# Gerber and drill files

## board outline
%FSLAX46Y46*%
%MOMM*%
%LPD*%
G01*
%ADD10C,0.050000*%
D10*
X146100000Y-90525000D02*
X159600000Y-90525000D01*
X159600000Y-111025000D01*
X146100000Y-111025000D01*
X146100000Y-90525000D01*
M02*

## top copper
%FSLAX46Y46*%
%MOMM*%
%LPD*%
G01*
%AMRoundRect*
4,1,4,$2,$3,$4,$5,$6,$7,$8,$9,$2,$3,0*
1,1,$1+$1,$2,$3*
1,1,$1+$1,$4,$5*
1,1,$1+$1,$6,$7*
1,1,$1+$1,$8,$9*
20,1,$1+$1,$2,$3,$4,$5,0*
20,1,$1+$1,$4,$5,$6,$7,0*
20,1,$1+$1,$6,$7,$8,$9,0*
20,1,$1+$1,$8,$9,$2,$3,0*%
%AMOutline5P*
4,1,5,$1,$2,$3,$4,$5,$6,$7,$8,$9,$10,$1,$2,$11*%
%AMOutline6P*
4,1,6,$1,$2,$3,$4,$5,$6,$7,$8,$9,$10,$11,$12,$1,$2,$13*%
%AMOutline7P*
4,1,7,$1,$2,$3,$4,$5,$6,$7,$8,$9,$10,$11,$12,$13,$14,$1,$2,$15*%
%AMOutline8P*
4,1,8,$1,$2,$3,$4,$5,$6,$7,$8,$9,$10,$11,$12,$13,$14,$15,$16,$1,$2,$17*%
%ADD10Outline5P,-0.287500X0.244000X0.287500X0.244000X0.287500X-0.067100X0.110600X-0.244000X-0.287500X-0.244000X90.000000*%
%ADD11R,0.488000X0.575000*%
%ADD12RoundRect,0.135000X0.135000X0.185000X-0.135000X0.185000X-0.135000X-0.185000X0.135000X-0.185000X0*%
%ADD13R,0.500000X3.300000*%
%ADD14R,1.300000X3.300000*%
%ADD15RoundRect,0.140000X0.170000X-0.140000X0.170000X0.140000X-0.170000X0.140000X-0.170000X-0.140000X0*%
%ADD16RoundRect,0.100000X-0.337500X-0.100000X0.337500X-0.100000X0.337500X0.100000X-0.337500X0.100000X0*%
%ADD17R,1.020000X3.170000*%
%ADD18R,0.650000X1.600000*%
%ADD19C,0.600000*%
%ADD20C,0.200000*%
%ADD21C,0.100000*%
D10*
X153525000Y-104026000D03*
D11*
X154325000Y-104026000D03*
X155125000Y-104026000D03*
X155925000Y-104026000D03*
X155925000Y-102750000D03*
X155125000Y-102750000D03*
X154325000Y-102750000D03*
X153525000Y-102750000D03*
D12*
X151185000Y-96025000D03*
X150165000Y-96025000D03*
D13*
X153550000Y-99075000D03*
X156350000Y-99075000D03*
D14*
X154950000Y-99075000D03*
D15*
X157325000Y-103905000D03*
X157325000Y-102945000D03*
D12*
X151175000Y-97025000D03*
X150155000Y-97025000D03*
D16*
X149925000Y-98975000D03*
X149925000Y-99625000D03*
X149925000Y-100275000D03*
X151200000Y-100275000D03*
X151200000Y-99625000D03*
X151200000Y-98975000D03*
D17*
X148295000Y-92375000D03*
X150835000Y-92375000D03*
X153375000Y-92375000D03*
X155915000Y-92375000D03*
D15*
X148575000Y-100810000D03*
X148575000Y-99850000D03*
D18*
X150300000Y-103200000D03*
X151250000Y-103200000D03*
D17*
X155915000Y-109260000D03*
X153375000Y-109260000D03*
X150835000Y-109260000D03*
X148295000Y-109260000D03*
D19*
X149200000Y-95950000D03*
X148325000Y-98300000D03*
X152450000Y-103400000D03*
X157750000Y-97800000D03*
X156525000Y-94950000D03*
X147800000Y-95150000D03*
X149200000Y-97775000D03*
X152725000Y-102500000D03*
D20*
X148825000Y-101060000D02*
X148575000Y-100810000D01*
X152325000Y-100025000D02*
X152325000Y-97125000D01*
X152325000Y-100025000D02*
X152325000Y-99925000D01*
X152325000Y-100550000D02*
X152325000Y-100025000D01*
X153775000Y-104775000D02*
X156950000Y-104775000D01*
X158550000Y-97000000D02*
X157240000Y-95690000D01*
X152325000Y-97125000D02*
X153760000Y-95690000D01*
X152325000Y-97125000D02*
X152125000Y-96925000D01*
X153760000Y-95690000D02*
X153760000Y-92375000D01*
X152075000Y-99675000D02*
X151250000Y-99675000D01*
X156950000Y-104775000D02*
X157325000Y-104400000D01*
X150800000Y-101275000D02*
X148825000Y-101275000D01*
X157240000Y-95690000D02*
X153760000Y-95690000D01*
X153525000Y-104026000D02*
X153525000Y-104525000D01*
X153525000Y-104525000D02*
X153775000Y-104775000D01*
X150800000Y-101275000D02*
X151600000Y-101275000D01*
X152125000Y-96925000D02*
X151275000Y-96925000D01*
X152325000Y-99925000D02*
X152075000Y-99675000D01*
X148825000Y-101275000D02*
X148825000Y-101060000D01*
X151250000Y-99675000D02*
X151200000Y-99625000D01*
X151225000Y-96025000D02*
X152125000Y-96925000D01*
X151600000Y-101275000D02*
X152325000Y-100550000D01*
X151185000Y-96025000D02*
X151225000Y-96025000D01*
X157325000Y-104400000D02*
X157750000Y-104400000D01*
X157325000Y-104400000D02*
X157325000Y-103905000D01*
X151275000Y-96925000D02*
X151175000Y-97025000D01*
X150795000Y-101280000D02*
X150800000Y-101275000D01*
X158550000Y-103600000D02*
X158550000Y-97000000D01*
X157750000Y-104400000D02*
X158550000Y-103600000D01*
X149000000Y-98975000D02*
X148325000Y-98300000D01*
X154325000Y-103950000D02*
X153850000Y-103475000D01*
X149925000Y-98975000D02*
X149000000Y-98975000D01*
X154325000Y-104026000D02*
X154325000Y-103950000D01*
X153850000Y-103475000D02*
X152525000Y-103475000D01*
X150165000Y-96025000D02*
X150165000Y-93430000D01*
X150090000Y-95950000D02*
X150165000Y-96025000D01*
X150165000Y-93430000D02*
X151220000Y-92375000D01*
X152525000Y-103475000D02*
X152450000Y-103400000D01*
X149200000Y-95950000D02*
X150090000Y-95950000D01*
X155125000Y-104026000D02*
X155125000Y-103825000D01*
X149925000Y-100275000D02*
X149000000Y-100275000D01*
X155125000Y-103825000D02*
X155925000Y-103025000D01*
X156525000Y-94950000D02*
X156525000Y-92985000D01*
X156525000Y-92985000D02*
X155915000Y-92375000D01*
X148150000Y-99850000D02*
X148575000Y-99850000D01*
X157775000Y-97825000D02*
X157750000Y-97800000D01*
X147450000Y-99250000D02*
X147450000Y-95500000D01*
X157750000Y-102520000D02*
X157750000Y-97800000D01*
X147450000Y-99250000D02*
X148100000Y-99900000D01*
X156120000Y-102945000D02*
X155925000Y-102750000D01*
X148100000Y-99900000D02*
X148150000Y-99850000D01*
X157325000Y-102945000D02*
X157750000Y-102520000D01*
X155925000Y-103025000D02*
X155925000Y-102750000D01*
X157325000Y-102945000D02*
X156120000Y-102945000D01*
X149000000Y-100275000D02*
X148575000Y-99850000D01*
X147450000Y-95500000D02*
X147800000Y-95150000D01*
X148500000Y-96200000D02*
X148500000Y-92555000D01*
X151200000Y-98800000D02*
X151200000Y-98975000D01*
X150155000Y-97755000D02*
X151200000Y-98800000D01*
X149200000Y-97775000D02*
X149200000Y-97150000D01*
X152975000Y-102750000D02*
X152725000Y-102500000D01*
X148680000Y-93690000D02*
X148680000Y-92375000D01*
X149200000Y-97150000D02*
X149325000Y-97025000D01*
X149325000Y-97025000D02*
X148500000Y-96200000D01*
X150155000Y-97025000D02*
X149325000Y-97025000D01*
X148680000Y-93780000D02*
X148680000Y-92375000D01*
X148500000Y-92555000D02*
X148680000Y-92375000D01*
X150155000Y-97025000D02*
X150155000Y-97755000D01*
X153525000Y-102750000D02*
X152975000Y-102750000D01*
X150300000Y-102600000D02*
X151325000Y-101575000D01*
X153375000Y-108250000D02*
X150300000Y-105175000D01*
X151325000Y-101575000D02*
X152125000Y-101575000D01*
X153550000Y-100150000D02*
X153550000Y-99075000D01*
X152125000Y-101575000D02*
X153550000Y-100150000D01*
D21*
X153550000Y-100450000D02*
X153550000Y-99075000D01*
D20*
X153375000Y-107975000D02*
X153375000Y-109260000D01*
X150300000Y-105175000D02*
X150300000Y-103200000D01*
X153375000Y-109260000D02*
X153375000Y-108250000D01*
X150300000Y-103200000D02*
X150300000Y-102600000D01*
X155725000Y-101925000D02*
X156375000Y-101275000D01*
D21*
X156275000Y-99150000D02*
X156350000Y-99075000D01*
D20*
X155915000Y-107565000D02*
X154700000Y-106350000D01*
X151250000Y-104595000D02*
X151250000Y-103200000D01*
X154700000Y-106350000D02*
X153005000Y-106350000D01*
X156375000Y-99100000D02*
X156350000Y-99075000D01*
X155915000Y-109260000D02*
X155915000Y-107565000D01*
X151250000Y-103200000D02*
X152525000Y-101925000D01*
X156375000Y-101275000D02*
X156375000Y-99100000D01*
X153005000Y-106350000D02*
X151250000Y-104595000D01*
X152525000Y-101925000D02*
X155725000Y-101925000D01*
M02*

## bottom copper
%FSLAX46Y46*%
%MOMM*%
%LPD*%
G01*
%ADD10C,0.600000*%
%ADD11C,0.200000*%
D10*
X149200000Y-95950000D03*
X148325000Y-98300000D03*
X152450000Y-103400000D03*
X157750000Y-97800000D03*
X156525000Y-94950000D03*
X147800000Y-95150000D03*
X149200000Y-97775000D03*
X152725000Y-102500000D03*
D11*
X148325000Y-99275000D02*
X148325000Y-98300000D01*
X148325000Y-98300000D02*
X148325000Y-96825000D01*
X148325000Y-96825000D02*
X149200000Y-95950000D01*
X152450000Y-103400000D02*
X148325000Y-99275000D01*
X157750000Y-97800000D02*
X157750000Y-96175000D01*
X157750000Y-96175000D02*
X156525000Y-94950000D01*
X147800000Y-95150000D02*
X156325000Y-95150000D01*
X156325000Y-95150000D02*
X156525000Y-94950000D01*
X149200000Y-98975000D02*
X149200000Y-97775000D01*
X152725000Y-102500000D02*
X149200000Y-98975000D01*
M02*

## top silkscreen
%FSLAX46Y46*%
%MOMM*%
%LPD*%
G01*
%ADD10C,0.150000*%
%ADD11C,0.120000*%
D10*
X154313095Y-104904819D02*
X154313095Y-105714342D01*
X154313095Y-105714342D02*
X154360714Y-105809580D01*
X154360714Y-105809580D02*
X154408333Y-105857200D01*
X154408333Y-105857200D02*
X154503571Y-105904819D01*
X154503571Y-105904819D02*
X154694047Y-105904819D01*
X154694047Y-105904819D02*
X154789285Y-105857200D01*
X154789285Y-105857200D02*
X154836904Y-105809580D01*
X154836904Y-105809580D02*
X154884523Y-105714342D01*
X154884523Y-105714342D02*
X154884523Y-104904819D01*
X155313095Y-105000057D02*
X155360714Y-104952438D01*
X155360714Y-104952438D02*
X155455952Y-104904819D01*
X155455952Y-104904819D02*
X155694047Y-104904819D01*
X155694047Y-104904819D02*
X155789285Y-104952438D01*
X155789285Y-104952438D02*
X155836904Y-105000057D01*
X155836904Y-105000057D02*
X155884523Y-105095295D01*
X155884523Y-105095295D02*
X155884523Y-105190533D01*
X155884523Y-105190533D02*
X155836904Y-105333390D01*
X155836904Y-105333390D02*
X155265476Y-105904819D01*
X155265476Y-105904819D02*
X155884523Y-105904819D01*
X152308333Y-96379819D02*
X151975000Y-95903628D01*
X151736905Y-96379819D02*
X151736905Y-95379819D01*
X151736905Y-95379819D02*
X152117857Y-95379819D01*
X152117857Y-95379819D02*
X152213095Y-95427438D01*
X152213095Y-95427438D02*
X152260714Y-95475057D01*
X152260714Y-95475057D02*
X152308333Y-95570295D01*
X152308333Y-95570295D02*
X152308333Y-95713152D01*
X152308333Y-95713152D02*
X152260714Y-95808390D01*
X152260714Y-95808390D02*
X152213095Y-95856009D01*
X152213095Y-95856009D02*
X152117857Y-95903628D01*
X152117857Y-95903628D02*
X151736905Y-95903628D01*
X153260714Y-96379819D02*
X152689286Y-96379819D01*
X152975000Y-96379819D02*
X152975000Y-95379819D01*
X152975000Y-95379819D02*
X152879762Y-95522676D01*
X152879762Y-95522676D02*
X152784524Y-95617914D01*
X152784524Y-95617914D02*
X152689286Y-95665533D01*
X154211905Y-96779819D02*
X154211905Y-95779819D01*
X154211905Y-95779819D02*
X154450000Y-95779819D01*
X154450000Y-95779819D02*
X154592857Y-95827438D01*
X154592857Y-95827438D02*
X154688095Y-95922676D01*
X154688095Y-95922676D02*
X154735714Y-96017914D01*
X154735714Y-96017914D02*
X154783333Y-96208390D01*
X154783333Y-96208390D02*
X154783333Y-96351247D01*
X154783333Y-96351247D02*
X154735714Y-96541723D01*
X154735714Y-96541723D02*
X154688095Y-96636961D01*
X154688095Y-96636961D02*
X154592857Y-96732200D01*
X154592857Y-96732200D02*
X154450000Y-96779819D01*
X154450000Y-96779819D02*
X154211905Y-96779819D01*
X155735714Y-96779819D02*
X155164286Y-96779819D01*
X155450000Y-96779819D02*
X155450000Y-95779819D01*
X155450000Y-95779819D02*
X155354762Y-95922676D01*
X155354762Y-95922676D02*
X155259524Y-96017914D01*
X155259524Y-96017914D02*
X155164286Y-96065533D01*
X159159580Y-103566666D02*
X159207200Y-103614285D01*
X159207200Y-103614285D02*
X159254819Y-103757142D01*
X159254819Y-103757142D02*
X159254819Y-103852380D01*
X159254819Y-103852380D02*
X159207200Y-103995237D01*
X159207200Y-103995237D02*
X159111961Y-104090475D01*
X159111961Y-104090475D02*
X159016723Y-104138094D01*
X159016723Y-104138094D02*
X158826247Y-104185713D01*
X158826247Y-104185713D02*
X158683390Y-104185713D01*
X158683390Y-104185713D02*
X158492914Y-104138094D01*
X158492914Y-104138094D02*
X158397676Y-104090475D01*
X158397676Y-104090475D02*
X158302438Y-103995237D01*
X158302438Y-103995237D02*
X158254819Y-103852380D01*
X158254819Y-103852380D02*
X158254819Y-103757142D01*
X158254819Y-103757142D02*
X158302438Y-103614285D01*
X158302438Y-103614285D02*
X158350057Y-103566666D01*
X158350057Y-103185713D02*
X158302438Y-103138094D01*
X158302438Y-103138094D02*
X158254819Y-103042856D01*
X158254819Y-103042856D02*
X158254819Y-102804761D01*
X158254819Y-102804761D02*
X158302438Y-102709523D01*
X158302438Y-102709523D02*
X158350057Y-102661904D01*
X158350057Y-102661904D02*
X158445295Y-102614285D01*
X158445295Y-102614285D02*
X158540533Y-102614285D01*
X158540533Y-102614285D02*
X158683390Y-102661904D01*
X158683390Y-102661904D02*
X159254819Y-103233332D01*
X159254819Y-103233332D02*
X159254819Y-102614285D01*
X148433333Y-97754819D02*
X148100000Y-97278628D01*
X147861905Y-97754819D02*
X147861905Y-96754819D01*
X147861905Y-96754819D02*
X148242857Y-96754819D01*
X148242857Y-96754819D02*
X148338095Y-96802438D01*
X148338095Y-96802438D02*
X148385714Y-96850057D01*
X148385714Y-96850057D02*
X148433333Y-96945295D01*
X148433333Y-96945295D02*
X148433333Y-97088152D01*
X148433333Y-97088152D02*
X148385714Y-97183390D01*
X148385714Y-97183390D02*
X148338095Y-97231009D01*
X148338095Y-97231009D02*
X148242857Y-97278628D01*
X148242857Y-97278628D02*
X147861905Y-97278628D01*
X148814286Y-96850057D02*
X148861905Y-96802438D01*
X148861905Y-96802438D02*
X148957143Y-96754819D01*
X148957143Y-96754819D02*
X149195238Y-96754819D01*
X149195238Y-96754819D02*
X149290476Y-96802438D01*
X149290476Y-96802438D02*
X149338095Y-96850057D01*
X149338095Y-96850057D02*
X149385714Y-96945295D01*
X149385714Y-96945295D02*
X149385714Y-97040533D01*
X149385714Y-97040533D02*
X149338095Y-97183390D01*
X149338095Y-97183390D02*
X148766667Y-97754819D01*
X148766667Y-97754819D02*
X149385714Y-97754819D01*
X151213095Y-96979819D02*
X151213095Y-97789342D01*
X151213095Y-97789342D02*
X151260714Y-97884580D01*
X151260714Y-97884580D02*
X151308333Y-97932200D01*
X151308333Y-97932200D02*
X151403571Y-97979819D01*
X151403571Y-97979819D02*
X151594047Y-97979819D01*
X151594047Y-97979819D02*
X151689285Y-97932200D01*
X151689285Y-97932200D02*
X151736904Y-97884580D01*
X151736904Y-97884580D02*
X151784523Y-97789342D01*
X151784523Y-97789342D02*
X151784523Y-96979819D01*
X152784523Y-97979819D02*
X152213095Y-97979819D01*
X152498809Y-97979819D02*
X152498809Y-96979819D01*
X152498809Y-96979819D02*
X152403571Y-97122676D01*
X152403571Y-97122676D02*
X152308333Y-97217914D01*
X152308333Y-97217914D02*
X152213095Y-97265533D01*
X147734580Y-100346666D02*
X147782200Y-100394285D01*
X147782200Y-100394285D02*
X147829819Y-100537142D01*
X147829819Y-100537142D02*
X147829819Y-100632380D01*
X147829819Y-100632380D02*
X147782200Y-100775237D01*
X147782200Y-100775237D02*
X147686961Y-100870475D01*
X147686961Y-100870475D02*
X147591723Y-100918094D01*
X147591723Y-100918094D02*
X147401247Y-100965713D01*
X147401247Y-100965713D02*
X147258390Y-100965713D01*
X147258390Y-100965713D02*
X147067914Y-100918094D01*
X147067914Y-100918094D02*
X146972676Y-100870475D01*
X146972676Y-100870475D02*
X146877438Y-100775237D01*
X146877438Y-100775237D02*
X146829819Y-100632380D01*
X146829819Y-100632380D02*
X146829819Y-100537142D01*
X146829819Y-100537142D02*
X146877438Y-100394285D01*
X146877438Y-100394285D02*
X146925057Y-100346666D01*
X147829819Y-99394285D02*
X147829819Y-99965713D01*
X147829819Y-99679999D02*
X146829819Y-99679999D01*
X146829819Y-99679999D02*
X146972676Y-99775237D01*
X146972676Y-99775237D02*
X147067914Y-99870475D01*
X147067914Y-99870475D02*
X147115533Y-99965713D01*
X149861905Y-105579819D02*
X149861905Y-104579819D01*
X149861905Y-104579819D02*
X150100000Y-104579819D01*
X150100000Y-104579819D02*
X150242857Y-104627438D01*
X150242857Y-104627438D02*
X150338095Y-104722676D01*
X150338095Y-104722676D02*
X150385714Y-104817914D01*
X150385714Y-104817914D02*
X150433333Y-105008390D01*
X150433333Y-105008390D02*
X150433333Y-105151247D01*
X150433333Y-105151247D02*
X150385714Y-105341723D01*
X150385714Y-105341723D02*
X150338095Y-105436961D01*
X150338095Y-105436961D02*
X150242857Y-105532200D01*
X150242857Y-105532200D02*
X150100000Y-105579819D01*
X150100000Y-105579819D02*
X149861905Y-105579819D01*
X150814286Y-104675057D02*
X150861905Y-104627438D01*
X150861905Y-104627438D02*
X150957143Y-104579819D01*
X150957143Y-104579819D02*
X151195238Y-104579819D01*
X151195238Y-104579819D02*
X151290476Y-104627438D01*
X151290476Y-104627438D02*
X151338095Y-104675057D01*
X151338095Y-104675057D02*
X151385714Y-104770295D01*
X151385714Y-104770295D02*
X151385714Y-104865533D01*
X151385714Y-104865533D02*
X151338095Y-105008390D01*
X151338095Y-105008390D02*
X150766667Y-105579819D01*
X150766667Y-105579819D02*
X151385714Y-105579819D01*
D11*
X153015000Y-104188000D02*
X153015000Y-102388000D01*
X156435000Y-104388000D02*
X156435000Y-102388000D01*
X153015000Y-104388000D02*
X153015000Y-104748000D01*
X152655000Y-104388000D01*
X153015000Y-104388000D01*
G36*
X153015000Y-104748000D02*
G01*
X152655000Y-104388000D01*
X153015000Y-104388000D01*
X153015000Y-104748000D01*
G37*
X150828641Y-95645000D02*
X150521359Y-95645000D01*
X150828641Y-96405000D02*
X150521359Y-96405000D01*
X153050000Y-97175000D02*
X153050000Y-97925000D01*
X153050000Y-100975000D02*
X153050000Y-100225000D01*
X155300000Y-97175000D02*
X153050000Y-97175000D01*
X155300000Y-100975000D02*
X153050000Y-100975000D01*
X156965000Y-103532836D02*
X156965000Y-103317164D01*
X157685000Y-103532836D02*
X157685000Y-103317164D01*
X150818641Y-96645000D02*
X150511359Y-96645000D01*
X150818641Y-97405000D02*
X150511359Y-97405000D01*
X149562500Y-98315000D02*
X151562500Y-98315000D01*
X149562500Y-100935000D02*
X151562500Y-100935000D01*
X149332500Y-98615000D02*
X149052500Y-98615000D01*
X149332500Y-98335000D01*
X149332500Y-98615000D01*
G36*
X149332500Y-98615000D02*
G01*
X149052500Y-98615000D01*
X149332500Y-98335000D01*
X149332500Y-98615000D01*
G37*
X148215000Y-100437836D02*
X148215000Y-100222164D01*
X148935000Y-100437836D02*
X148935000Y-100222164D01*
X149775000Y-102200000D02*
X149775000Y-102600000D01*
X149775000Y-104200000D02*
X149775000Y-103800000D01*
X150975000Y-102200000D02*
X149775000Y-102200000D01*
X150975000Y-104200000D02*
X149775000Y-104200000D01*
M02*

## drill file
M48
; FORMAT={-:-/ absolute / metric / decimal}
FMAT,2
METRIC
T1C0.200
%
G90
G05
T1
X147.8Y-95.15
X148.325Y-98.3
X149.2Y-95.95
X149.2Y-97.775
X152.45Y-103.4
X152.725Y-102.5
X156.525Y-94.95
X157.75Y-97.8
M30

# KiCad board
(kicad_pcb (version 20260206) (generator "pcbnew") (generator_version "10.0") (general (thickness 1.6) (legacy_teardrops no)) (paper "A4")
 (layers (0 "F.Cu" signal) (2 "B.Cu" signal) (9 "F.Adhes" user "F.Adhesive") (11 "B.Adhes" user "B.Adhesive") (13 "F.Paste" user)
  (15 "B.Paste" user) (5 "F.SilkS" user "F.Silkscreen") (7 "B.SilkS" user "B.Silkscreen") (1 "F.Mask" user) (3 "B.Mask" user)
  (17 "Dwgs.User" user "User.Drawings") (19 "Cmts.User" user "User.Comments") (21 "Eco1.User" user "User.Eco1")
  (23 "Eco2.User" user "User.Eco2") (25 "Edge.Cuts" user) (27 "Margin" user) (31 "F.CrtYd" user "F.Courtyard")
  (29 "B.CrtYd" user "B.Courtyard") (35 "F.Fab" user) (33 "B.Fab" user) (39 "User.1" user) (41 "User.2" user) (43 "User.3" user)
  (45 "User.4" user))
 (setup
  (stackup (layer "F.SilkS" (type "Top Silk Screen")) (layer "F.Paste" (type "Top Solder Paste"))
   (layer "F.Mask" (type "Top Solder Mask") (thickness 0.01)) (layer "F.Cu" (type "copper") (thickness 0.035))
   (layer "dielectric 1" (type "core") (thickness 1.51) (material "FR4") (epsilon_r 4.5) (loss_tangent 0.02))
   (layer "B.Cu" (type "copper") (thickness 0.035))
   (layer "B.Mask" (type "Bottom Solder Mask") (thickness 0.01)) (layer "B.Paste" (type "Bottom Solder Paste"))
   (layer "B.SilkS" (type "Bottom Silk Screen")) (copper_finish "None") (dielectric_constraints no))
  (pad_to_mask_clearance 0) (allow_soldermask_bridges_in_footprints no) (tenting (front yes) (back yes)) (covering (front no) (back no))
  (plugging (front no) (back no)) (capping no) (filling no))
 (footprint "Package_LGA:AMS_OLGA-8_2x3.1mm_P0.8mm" (layer "F.Cu") (at 154.725 103.388 90)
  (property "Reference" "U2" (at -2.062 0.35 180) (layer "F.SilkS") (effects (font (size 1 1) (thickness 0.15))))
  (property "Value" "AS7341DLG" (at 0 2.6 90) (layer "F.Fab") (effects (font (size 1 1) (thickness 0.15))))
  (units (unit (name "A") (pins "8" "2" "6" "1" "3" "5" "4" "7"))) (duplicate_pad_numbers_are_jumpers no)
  (fp_line (start -0.8 -1.71) (end 1 -1.71) (stroke (width 0.12) (type solid)) (layer "F.SilkS"))
  (fp_line (start -1 1.71) (end 1 1.71) (stroke (width 0.12) (type solid)) (layer "F.SilkS"))
  (fp_poly (pts (xy -1 -1.71) (xy -1.36 -1.71) (xy -1 -2.07) (xy -1 -1.71)) (stroke (width 0.12) (type solid)) (fill yes) (layer "F.SilkS"))
  (pad "1" smd roundrect (at -0.638 -1.2 90) (size 0.575 0.488) (layers "F.Cu" "F.Mask" "F.Paste") (roundrect_rratio 0)
   (chamfer_ratio 0.3625) (chamfer bottom_right) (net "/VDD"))
  (pad "2" smd rect (at -0.638 -0.4 90) (size 0.575 0.488) (layers "F.Cu" "F.Mask" "F.Paste") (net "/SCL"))
  (pad "3" smd rect (at -0.638 0.4 90) (size 0.575 0.488) (layers "F.Cu" "F.Mask" "F.Paste") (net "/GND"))
  (pad "4" smd rect (at -0.638 1.2 90) (size 0.575 0.488) (layers "F.Cu" "F.Mask" "F.Paste") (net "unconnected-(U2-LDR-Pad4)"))
  (pad "5" smd rect (at 0.638 1.2 90) (size 0.575 0.488) (layers "F.Cu" "F.Mask" "F.Paste") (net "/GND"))
  (pad "6" smd rect (at 0.638 0.4 90) (size 0.575 0.488) (layers "F.Cu" "F.Mask" "F.Paste") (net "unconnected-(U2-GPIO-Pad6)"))
  (pad "7" smd rect (at 0.638 -0.4 90) (size 0.575 0.488) (layers "F.Cu" "F.Mask" "F.Paste") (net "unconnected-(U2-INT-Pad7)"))
  (pad "8" smd rect (at 0.638 -1.2 90) (size 0.575 0.488) (layers "F.Cu" "F.Mask" "F.Paste") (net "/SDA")))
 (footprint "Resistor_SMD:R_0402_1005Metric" (layer "F.Cu") (at 150.675 96.025 180)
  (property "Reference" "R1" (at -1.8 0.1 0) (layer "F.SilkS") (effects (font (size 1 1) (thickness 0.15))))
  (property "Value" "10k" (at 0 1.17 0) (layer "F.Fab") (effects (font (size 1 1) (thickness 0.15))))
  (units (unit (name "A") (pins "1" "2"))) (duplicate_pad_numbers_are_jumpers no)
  (fp_line (start -0.153641 0.38) (end 0.153641 0.38) (stroke (width 0.12) (type solid)) (layer "F.SilkS"))
  (fp_line (start -0.153641 -0.38) (end 0.153641 -0.38) (stroke (width 0.12) (type solid)) (layer "F.SilkS"))
  (pad "1" smd roundrect (at -0.51 0 180) (size 0.54 0.64) (layers "F.Cu" "F.Mask" "F.Paste") (roundrect_rratio 0.25) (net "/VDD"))
  (pad "2" smd roundrect (at 0.51 0 180) (size 0.54 0.64) (layers "F.Cu" "F.Mask" "F.Paste") (roundrect_rratio 0.25) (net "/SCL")))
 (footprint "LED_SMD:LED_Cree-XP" (layer "F.Cu") (at 154.95 99.075)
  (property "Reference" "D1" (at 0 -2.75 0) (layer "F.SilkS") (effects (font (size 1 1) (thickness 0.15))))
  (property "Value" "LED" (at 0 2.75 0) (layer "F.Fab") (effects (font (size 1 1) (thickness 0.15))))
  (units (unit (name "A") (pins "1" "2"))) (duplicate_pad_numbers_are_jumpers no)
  (fp_line (start -1.9 -1.9) (end -1.9 -1.15) (stroke (width 0.12) (type solid)) (layer "F.SilkS"))
  (fp_line (start -1.9 1.9) (end -1.9 1.15) (stroke (width 0.12) (type solid)) (layer "F.SilkS"))
  (fp_line (start 0.35 -1.9) (end -1.9 -1.9) (stroke (width 0.12) (type solid)) (layer "F.SilkS"))
  (fp_line (start 0.35 1.9) (end -1.9 1.9) (stroke (width 0.12) (type solid)) (layer "F.SilkS"))
  (pad "" smd rect (at 0 -1) (size 1.01 0.75) (layers "F.Paste"))
  (pad "" smd rect (at 0 0) (size 1.01 0.75) (layers "F.Paste"))
  (pad "" smd rect (at 0 1) (size 1.01 0.75) (layers "F.Paste"))
  (pad "1" smd rect (at -1.4 0) (size 0.5 3.3) (layers "F.Cu" "F.Mask" "F.Paste") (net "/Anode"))
  (pad "2" smd rect (at 1.4 0) (size 0.5 3.3) (layers "F.Cu" "F.Mask" "F.Paste") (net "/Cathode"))
  (pad "3" smd rect (at 0 0) (size 1.3 3.3) (layers "F.Cu" "F.Mask")))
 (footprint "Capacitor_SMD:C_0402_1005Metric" (layer "F.Cu") (at 157.325 103.425 90)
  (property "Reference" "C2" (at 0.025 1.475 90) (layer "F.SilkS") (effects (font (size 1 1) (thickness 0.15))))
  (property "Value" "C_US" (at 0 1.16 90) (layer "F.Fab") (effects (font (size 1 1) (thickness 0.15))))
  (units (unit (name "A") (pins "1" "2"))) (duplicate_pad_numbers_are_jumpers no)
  (fp_line (start -0.107836 -0.36) (end 0.107836 -0.36) (stroke (width 0.12) (type solid)) (layer "F.SilkS"))
  (fp_line (start -0.107836 0.36) (end 0.107836 0.36) (stroke (width 0.12) (type solid)) (layer "F.SilkS"))
  (pad "1" smd roundrect (at -0.48 0 90) (size 0.56 0.62) (layers "F.Cu" "F.Mask" "F.Paste") (roundrect_rratio 0.25) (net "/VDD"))
  (pad "2" smd roundrect (at 0.48 0 90) (size 0.56 0.62) (layers "F.Cu" "F.Mask" "F.Paste") (roundrect_rratio 0.25) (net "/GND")))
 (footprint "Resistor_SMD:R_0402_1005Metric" (layer "F.Cu") (at 150.665 97.025 180)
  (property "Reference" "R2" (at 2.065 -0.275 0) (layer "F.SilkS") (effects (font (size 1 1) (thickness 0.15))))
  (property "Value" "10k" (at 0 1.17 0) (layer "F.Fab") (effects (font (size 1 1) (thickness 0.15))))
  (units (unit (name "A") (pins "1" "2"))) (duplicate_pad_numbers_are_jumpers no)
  (fp_line (start -0.153641 0.38) (end 0.153641 0.38) (stroke (width 0.12) (type solid)) (layer "F.SilkS"))
  (fp_line (start -0.153641 -0.38) (end 0.153641 -0.38) (stroke (width 0.12) (type solid)) (layer "F.SilkS"))
  (pad "1" smd roundrect (at -0.51 0 180) (size 0.54 0.64) (layers "F.Cu" "F.Mask" "F.Paste") (roundrect_rratio 0.25) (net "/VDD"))
  (pad "2" smd roundrect (at 0.51 0 180) (size 0.54 0.64) (layers "F.Cu" "F.Mask" "F.Paste") (roundrect_rratio 0.25) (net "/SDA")))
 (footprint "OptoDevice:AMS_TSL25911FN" (layer "F.Cu") (at 150.5625 99.625)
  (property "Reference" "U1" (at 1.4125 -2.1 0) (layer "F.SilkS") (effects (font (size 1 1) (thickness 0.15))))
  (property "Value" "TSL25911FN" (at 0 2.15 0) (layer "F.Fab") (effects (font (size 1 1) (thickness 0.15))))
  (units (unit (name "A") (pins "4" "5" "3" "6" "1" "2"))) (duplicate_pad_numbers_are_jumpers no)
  (fp_line (start -1 -1.31) (end 1 -1.31) (stroke (width 0.12) (type solid)) (layer "F.SilkS"))
  (fp_line (start -1 1.31) (end 1 1.31) (stroke (width 0.12) (type solid)) (layer "F.SilkS"))
  (fp_poly
   (pts (xy -1.23 -1.01) (xy -1.51 -1.01) (xy -1.23 -1.29) (xy -1.23 -1.01)) (stroke (width 0.12) (type solid)) (fill yes) (layer "F.SilkS"))
  (pad "1" smd roundrect (at -0.6375 -0.65) (size 0.875 0.4) (layers "F.Cu" "F.Mask" "F.Paste") (roundrect_rratio 0.25) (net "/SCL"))
  (pad "2" smd roundrect (at -0.6375 0) (size 0.875 0.4) (layers "F.Cu" "F.Mask" "F.Paste") (roundrect_rratio 0.25)
   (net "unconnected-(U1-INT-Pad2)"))
  (pad "3" smd roundrect (at -0.6375 0.65) (size 0.875 0.4) (layers "F.Cu" "F.Mask" "F.Paste") (roundrect_rratio 0.25) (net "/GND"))
  (pad "4" smd roundrect (at 0.6375 0.65) (size 0.875 0.4) (layers "F.Cu" "F.Mask" "F.Paste") (roundrect_rratio 0.25)
   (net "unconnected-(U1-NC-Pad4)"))
  (pad "5" smd roundrect (at 0.6375 0) (size 0.875 0.4) (layers "F.Cu" "F.Mask" "F.Paste") (roundrect_rratio 0.25) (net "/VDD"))
  (pad "6" smd roundrect (at 0.6375 -0.65) (size 0.875 0.4) (layers "F.Cu" "F.Mask" "F.Paste") (roundrect_rratio 0.25) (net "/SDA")))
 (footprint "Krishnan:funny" (layer "F.Cu") (at 147.973012 109.725 90)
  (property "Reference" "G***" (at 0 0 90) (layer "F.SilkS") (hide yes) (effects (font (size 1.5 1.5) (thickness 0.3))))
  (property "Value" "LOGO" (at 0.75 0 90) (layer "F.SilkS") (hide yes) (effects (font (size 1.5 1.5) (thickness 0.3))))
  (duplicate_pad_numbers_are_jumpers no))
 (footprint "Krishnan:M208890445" (layer "F.Cu") (at 152.105 88.76)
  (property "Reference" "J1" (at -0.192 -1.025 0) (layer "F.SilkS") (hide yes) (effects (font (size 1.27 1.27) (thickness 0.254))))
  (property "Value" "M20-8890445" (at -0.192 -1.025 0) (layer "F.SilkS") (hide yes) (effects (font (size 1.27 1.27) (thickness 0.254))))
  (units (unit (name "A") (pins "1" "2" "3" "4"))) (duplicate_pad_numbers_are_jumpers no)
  (pad "1" smd rect (at -3.81 3.615) (size 1.02 3.17) (layers "F.Cu" "F.Mask" "F.Paste") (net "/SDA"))
  (pad "2" smd rect (at -1.27 3.615) (size 1.02 3.17) (layers "F.Cu" "F.Mask" "F.Paste") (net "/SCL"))
  (pad "3" smd rect (at 1.27 3.615) (size 1.02 3.17) (layers "F.Cu" "F.Mask" "F.Paste") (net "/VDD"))
  (pad "4" smd rect (at 3.81 3.615) (size 1.02 3.17) (layers "F.Cu" "F.Mask" "F.Paste") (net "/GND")))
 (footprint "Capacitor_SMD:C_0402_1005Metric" (layer "F.Cu") (at 148.575 100.33 90)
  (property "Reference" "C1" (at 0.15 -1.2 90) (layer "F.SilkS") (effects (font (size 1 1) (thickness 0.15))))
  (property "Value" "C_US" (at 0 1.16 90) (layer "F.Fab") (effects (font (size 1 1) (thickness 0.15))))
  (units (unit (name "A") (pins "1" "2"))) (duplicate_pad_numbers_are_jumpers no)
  (fp_line (start -0.107836 -0.36) (end 0.107836 -0.36) (stroke (width 0.12) (type solid)) (layer "F.SilkS"))
  (fp_line (start -0.107836 0.36) (end 0.107836 0.36) (stroke (width 0.12) (type solid)) (layer "F.SilkS"))
  (pad "1" smd roundrect (at -0.48 0 90) (size 0.56 0.62) (layers "F.Cu" "F.Mask" "F.Paste") (roundrect_rratio 0.25) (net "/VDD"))
  (pad "2" smd roundrect (at 0.48 0 90) (size 0.56 0.62) (layers "F.Cu" "F.Mask" "F.Paste") (roundrect_rratio 0.25) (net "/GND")))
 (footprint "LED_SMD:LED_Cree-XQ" (layer "F.Cu") (at 150.775 103.2)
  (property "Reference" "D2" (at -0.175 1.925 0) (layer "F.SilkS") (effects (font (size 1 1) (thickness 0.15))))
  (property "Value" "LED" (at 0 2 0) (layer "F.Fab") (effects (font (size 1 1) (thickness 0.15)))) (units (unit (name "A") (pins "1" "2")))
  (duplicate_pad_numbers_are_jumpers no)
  (fp_line (start -1 -1) (end -1 -0.6) (stroke (width 0.12) (type solid)) (layer "F.SilkS"))
  (fp_line (start -1 1) (end -1 0.6) (stroke (width 0.12) (type solid)) (layer "F.SilkS"))
  (fp_line (start 0.2 -1) (end -1 -1) (stroke (width 0.12) (type solid)) (layer "F.SilkS"))
  (fp_line (start 0.2 1) (end -1 1) (stroke (width 0.12) (type solid)) (layer "F.SilkS"))
  (pad "1" smd rect (at -0.475 0) (size 0.65 1.6) (layers "F.Cu" "F.Mask" "F.Paste") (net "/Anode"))
  (pad "2" smd rect (at 0.475 0) (size 0.65 1.6) (layers "F.Cu" "F.Mask" "F.Paste") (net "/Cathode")))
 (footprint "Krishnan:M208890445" (layer "F.Cu") (at 152.105 112.875 180)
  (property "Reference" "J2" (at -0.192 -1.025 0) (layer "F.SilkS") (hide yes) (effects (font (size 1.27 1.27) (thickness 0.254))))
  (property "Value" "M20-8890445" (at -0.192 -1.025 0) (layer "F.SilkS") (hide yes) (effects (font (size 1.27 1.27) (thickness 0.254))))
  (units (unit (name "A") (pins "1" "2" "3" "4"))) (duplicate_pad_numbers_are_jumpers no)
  (pad "1" smd rect (at -3.81 3.615 180) (size 1.02 3.17) (layers "F.Cu" "F.Mask" "F.Paste") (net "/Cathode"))
  (pad "2" smd rect (at -1.27 3.615 180) (size 1.02 3.17) (layers "F.Cu" "F.Mask" "F.Paste") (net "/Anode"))
  (pad "3" smd rect (at 1.27 3.615 180) (size 1.02 3.17) (layers "F.Cu" "F.Mask" "F.Paste") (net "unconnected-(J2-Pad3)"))
  (pad "4" smd rect (at 3.81 3.615 180) (size 1.02 3.17) (layers "F.Cu" "F.Mask" "F.Paste") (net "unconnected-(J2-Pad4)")))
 (gr_rect (start 146.1 90.525) (end 159.6 111.025) (stroke (width 0.05) (type default)) (fill no) (layer "Edge.Cuts"))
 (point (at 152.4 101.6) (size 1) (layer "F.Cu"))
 (segment (start 148.825 101.06) (end 148.575 100.81) (width 0.2) (layer "F.Cu") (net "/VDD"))
 (segment (start 152.325 100.025) (end 152.325 97.125) (width 0.2) (layer "F.Cu") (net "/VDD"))
 (segment (start 152.325 100.025) (end 152.325 99.925) (width 0.2) (layer "F.Cu") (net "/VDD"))
 (segment (start 152.325 100.55) (end 152.325 100.025) (width 0.2) (layer "F.Cu") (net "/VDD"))
 (segment (start 153.775 104.775) (end 156.95 104.775) (width 0.2) (layer "F.Cu") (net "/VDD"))
 (segment (start 158.55 97) (end 157.24 95.69) (width 0.2) (layer "F.Cu") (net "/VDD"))
 (segment (start 152.325 97.125) (end 153.76 95.69) (width 0.2) (layer "F.Cu") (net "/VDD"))
 (segment (start 152.325 97.125) (end 152.125 96.925) (width 0.2) (layer "F.Cu") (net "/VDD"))
 (segment (start 153.76 95.69) (end 153.76 92.375) (width 0.2) (layer "F.Cu") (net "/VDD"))
 (segment (start 152.075 99.675) (end 151.25 99.675) (width 0.2) (layer "F.Cu") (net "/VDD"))
 (segment (start 156.95 104.775) (end 157.325 104.4) (width 0.2) (layer "F.Cu") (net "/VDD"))
 (segment (start 150.8 101.275) (end 148.825 101.275) (width 0.2) (layer "F.Cu") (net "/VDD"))
 (segment (start 157.24 95.69) (end 153.76 95.69) (width 0.2) (layer "F.Cu") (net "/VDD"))
 (segment (start 153.525 104.026) (end 153.525 104.525) (width 0.2) (layer "F.Cu") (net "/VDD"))
 (segment (start 153.525 104.525) (end 153.775 104.775) (width 0.2) (layer "F.Cu") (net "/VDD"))
 (segment (start 150.8 101.275) (end 151.6 101.275) (width 0.2) (layer "F.Cu") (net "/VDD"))
 (segment (start 152.125 96.925) (end 151.275 96.925) (width 0.2) (layer "F.Cu") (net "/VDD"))
 (segment (start 152.325 99.925) (end 152.075 99.675) (width 0.2) (layer "F.Cu") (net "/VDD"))
 (segment (start 148.825 101.275) (end 148.825 101.06) (width 0.2) (layer "F.Cu") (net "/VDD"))
 (segment (start 151.25 99.675) (end 151.2 99.625) (width 0.2) (layer "F.Cu") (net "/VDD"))
 (segment (start 151.225 96.025) (end 152.125 96.925) (width 0.2) (layer "F.Cu") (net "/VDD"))
 (segment (start 151.6 101.275) (end 152.325 100.55) (width 0.2) (layer "F.Cu") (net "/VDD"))
 (segment (start 151.185 96.025) (end 151.225 96.025) (width 0.2) (layer "F.Cu") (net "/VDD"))
 (segment (start 157.325 104.4) (end 157.75 104.4) (width 0.2) (layer "F.Cu") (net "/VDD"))
 (segment (start 157.325 104.4) (end 157.325 103.905) (width 0.2) (layer "F.Cu") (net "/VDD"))
 (segment (start 151.275 96.925) (end 151.175 97.025) (width 0.2) (layer "F.Cu") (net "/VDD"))
 (segment (start 150.795 101.28) (end 150.8 101.275) (width 0.2) (layer "F.Cu") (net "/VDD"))
 (segment (start 158.55 103.6) (end 158.55 97) (width 0.2) (layer "F.Cu") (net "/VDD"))
 (segment (start 157.75 104.4) (end 158.55 103.6) (width 0.2) (layer "F.Cu") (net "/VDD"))
 (segment (start 149 98.975) (end 148.325 98.3) (width 0.2) (layer "F.Cu") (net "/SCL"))
 (segment (start 154.325 103.95) (end 153.85 103.475) (width 0.2) (layer "F.Cu") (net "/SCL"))
 (segment (start 149.925 98.975) (end 149 98.975) (width 0.2) (layer "F.Cu") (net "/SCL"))
 (segment (start 154.325 104.026) (end 154.325 103.95) (width 0.2) (layer "F.Cu") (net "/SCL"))
 (segment (start 153.85 103.475) (end 152.525 103.475) (width 0.2) (layer "F.Cu") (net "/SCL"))
 (segment (start 150.165 96.025) (end 150.165 93.43) (width 0.2) (layer "F.Cu") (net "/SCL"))
 (segment (start 150.09 95.95) (end 150.165 96.025) (width 0.2) (layer "F.Cu") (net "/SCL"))
 (segment (start 150.165 93.43) (end 151.22 92.375) (width 0.2) (layer "F.Cu") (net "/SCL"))
 (segment (start 152.525 103.475) (end 152.45 103.4) (width 0.2) (layer "F.Cu") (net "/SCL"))
 (segment (start 149.2 95.95) (end 150.09 95.95) (width 0.2) (layer "F.Cu") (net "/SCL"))
 (via (at 149.2 95.95) (size 0.6) (drill 0.2) (layers "F.Cu" "B.Cu") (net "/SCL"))
 (via (at 148.325 98.3) (size 0.6) (drill 0.2) (layers "F.Cu" "B.Cu") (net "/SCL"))
 (via (at 152.45 103.4) (size 0.6) (drill 0.2) (layers "F.Cu" "B.Cu") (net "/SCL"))
 (segment (start 148.325 99.275) (end 148.325 98.3) (width 0.2) (layer "B.Cu") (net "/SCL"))
 (segment (start 148.325 98.3) (end 148.325 96.825) (width 0.2) (layer "B.Cu") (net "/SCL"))
 (segment (start 148.325 96.825) (end 149.2 95.95) (width 0.2) (layer "B.Cu") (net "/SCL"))
 (segment (start 152.45 103.4) (end 148.325 99.275) (width 0.2) (layer "B.Cu") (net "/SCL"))
 (segment (start 155.125 104.026) (end 155.125 103.825) (width 0.2) (layer "F.Cu") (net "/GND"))
 (segment (start 149.925 100.275) (end 149 100.275) (width 0.2) (layer "F.Cu") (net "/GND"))
 (segment (start 155.125 103.825) (end 155.925 103.025) (width 0.2) (layer "F.Cu") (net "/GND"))
 (segment (start 156.525 94.95) (end 156.525 92.985) (width 0.2) (layer "F.Cu") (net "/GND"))
 (segment (start 156.525 92.985) (end 155.915 92.375) (width 0.2) (layer "F.Cu") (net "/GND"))
 (segment (start 148.15 99.85) (end 148.575 99.85) (width 0.2) (layer "F.Cu") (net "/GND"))
 (segment (start 157.775 97.825) (end 157.75 97.8) (width 0.2) (layer "F.Cu") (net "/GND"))
 (segment (start 147.45 99.25) (end 147.45 95.5) (width 0.2) (layer "F.Cu") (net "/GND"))
 (segment (start 157.75 102.52) (end 157.75 97.8) (width 0.2) (layer "F.Cu") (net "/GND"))
 (segment (start 147.45 99.25) (end 148.1 99.9) (width 0.2) (layer "F.Cu") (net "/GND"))
 (segment (start 156.12 102.945) (end 155.925 102.75) (width 0.2) (layer "F.Cu") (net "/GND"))
 (segment (start 148.1 99.9) (end 148.15 99.85) (width 0.2) (layer "F.Cu") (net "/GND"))
 (segment (start 157.325 102.945) (end 157.75 102.52) (width 0.2) (layer "F.Cu") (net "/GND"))
 (segment (start 155.925 103.025) (end 155.925 102.75) (width 0.2) (layer "F.Cu") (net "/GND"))
 (segment (start 157.325 102.945) (end 156.12 102.945) (width 0.2) (layer "F.Cu") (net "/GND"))
 (segment (start 149 100.275) (end 148.575 99.85) (width 0.2) (layer "F.Cu") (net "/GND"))
 (segment (start 147.45 95.5) (end 147.8 95.15) (width 0.2) (layer "F.Cu") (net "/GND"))
 (via (at 157.75 97.8) (size 0.6) (drill 0.2) (layers "F.Cu" "B.Cu") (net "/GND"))
 (via (at 156.525 94.95) (size 0.6) (drill 0.2) (layers "F.Cu" "B.Cu") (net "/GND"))
 (via (at 147.8 95.15) (size 0.6) (drill 0.2) (layers "F.Cu" "B.Cu") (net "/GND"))
 (segment (start 157.75 97.8) (end 157.75 96.175) (width 0.2) (layer "B.Cu") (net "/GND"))
 (segment (start 157.75 96.175) (end 156.525 94.95) (width 0.2) (layer "B.Cu") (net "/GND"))
 (segment (start 147.8 95.15) (end 156.325 95.15) (width 0.2) (layer "B.Cu") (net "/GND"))
 (segment (start 156.325 95.15) (end 156.525 94.95) (width 0.2) (layer "B.Cu") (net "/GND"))
 (segment (start 148.5 96.2) (end 148.5 92.555) (width 0.2) (layer "F.Cu") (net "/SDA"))
 (segment (start 151.2 98.8) (end 151.2 98.975) (width 0.2) (layer "F.Cu") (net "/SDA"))
 (segment (start 150.155 97.755) (end 151.2 98.8) (width 0.2) (layer "F.Cu") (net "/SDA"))
 (segment (start 149.2 97.775) (end 149.2 97.15) (width 0.2) (layer "F.Cu") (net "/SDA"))
 (segment (start 152.975 102.75) (end 152.725 102.5) (width 0.2) (layer "F.Cu") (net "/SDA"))
 (segment (start 148.68 93.69) (end 148.68 92.375) (width 0.2) (layer "F.Cu") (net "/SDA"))
 (segment (start 149.2 97.15) (end 149.325 97.025) (width 0.2) (layer "F.Cu") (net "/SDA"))
 (segment (start 149.325 97.025) (end 148.5 96.2) (width 0.2) (layer "F.Cu") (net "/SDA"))
 (segment (start 150.155 97.025) (end 149.325 97.025) (width 0.2) (layer "F.Cu") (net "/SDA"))
 (segment (start 148.68 93.78) (end 148.68 92.375) (width 0.2) (layer "F.Cu") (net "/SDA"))
 (segment (start 148.5 92.555) (end 148.68 92.375) (width 0.2) (layer "F.Cu") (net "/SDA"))
 (segment (start 150.155 97.025) (end 150.155 97.755) (width 0.2) (layer "F.Cu") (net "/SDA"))
 (segment (start 153.525 102.75) (end 152.975 102.75) (width 0.2) (layer "F.Cu") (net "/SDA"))
 (via (at 149.2 97.775) (size 0.6) (drill 0.2) (layers "F.Cu" "B.Cu") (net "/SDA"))
 (via (at 152.725 102.5) (size 0.6) (drill 0.2) (layers "F.Cu" "B.Cu") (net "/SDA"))
 (segment (start 149.2 98.975) (end 149.2 97.775) (width 0.2) (layer "B.Cu") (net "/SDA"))
 (segment (start 152.725 102.5) (end 149.2 98.975) (width 0.2) (layer "B.Cu") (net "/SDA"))
 (segment (start 150.3 102.6) (end 151.325 101.575) (width 0.2) (layer "F.Cu") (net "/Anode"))
 (segment (start 153.375 108.25) (end 150.3 105.175) (width 0.2) (layer "F.Cu") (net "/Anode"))
 (segment (start 151.325 101.575) (end 152.125 101.575) (width 0.2) (layer "F.Cu") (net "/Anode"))
 (segment (start 153.55 100.15) (end 153.55 99.075) (width 0.2) (layer "F.Cu") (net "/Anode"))
 (segment (start 152.125 101.575) (end 153.55 100.15) (width 0.2) (layer "F.Cu") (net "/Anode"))
 (segment (start 153.55 100.45) (end 153.55 99.075) (width 0.1) (layer "F.Cu") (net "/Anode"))
 (segment (start 153.375 107.975) (end 153.375 109.26) (width 0.2) (layer "F.Cu") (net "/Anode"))
 (segment (start 150.3 105.175) (end 150.3 103.2) (width 0.2) (layer "F.Cu") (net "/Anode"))
 (segment (start 153.375 109.26) (end 153.375 108.25) (width 0.2) (layer "F.Cu") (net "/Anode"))
 (segment (start 150.3 103.2) (end 150.3 102.6) (width 0.2) (layer "F.Cu") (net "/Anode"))
 (segment (start 155.725 101.925) (end 156.375 101.275) (width 0.2) (layer "F.Cu") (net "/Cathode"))
 (segment (start 156.275 99.15) (end 156.35 99.075) (width 0.1) (layer "F.Cu") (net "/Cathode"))
 (segment (start 155.915 107.565) (end 154.7 106.35) (width 0.2) (layer "F.Cu") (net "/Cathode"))
 (segment (start 151.25 104.595) (end 151.25 103.2) (width 0.2) (layer "F.Cu") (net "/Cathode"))
 (segment (start 154.7 106.35) (end 153.005 106.35) (width 0.2) (layer "F.Cu") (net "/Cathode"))
 (segment (start 156.375 99.1) (end 156.35 99.075) (width 0.2) (layer "F.Cu") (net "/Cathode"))
 (segment (start 155.915 109.26) (end 155.915 107.565) (width 0.2) (layer "F.Cu") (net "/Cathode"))
 (segment (start 151.25 103.2) (end 152.525 101.925) (width 0.2) (layer "F.Cu") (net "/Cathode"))
 (segment (start 156.375 101.275) (end 156.375 99.1) (width 0.2) (layer "F.Cu") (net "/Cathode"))
 (segment (start 153.005 106.35) (end 151.25 104.595) (width 0.2) (layer "F.Cu") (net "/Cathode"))
 (segment (start 152.525 101.925) (end 155.725 101.925) (width 0.2) (layer "F.Cu") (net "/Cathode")))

